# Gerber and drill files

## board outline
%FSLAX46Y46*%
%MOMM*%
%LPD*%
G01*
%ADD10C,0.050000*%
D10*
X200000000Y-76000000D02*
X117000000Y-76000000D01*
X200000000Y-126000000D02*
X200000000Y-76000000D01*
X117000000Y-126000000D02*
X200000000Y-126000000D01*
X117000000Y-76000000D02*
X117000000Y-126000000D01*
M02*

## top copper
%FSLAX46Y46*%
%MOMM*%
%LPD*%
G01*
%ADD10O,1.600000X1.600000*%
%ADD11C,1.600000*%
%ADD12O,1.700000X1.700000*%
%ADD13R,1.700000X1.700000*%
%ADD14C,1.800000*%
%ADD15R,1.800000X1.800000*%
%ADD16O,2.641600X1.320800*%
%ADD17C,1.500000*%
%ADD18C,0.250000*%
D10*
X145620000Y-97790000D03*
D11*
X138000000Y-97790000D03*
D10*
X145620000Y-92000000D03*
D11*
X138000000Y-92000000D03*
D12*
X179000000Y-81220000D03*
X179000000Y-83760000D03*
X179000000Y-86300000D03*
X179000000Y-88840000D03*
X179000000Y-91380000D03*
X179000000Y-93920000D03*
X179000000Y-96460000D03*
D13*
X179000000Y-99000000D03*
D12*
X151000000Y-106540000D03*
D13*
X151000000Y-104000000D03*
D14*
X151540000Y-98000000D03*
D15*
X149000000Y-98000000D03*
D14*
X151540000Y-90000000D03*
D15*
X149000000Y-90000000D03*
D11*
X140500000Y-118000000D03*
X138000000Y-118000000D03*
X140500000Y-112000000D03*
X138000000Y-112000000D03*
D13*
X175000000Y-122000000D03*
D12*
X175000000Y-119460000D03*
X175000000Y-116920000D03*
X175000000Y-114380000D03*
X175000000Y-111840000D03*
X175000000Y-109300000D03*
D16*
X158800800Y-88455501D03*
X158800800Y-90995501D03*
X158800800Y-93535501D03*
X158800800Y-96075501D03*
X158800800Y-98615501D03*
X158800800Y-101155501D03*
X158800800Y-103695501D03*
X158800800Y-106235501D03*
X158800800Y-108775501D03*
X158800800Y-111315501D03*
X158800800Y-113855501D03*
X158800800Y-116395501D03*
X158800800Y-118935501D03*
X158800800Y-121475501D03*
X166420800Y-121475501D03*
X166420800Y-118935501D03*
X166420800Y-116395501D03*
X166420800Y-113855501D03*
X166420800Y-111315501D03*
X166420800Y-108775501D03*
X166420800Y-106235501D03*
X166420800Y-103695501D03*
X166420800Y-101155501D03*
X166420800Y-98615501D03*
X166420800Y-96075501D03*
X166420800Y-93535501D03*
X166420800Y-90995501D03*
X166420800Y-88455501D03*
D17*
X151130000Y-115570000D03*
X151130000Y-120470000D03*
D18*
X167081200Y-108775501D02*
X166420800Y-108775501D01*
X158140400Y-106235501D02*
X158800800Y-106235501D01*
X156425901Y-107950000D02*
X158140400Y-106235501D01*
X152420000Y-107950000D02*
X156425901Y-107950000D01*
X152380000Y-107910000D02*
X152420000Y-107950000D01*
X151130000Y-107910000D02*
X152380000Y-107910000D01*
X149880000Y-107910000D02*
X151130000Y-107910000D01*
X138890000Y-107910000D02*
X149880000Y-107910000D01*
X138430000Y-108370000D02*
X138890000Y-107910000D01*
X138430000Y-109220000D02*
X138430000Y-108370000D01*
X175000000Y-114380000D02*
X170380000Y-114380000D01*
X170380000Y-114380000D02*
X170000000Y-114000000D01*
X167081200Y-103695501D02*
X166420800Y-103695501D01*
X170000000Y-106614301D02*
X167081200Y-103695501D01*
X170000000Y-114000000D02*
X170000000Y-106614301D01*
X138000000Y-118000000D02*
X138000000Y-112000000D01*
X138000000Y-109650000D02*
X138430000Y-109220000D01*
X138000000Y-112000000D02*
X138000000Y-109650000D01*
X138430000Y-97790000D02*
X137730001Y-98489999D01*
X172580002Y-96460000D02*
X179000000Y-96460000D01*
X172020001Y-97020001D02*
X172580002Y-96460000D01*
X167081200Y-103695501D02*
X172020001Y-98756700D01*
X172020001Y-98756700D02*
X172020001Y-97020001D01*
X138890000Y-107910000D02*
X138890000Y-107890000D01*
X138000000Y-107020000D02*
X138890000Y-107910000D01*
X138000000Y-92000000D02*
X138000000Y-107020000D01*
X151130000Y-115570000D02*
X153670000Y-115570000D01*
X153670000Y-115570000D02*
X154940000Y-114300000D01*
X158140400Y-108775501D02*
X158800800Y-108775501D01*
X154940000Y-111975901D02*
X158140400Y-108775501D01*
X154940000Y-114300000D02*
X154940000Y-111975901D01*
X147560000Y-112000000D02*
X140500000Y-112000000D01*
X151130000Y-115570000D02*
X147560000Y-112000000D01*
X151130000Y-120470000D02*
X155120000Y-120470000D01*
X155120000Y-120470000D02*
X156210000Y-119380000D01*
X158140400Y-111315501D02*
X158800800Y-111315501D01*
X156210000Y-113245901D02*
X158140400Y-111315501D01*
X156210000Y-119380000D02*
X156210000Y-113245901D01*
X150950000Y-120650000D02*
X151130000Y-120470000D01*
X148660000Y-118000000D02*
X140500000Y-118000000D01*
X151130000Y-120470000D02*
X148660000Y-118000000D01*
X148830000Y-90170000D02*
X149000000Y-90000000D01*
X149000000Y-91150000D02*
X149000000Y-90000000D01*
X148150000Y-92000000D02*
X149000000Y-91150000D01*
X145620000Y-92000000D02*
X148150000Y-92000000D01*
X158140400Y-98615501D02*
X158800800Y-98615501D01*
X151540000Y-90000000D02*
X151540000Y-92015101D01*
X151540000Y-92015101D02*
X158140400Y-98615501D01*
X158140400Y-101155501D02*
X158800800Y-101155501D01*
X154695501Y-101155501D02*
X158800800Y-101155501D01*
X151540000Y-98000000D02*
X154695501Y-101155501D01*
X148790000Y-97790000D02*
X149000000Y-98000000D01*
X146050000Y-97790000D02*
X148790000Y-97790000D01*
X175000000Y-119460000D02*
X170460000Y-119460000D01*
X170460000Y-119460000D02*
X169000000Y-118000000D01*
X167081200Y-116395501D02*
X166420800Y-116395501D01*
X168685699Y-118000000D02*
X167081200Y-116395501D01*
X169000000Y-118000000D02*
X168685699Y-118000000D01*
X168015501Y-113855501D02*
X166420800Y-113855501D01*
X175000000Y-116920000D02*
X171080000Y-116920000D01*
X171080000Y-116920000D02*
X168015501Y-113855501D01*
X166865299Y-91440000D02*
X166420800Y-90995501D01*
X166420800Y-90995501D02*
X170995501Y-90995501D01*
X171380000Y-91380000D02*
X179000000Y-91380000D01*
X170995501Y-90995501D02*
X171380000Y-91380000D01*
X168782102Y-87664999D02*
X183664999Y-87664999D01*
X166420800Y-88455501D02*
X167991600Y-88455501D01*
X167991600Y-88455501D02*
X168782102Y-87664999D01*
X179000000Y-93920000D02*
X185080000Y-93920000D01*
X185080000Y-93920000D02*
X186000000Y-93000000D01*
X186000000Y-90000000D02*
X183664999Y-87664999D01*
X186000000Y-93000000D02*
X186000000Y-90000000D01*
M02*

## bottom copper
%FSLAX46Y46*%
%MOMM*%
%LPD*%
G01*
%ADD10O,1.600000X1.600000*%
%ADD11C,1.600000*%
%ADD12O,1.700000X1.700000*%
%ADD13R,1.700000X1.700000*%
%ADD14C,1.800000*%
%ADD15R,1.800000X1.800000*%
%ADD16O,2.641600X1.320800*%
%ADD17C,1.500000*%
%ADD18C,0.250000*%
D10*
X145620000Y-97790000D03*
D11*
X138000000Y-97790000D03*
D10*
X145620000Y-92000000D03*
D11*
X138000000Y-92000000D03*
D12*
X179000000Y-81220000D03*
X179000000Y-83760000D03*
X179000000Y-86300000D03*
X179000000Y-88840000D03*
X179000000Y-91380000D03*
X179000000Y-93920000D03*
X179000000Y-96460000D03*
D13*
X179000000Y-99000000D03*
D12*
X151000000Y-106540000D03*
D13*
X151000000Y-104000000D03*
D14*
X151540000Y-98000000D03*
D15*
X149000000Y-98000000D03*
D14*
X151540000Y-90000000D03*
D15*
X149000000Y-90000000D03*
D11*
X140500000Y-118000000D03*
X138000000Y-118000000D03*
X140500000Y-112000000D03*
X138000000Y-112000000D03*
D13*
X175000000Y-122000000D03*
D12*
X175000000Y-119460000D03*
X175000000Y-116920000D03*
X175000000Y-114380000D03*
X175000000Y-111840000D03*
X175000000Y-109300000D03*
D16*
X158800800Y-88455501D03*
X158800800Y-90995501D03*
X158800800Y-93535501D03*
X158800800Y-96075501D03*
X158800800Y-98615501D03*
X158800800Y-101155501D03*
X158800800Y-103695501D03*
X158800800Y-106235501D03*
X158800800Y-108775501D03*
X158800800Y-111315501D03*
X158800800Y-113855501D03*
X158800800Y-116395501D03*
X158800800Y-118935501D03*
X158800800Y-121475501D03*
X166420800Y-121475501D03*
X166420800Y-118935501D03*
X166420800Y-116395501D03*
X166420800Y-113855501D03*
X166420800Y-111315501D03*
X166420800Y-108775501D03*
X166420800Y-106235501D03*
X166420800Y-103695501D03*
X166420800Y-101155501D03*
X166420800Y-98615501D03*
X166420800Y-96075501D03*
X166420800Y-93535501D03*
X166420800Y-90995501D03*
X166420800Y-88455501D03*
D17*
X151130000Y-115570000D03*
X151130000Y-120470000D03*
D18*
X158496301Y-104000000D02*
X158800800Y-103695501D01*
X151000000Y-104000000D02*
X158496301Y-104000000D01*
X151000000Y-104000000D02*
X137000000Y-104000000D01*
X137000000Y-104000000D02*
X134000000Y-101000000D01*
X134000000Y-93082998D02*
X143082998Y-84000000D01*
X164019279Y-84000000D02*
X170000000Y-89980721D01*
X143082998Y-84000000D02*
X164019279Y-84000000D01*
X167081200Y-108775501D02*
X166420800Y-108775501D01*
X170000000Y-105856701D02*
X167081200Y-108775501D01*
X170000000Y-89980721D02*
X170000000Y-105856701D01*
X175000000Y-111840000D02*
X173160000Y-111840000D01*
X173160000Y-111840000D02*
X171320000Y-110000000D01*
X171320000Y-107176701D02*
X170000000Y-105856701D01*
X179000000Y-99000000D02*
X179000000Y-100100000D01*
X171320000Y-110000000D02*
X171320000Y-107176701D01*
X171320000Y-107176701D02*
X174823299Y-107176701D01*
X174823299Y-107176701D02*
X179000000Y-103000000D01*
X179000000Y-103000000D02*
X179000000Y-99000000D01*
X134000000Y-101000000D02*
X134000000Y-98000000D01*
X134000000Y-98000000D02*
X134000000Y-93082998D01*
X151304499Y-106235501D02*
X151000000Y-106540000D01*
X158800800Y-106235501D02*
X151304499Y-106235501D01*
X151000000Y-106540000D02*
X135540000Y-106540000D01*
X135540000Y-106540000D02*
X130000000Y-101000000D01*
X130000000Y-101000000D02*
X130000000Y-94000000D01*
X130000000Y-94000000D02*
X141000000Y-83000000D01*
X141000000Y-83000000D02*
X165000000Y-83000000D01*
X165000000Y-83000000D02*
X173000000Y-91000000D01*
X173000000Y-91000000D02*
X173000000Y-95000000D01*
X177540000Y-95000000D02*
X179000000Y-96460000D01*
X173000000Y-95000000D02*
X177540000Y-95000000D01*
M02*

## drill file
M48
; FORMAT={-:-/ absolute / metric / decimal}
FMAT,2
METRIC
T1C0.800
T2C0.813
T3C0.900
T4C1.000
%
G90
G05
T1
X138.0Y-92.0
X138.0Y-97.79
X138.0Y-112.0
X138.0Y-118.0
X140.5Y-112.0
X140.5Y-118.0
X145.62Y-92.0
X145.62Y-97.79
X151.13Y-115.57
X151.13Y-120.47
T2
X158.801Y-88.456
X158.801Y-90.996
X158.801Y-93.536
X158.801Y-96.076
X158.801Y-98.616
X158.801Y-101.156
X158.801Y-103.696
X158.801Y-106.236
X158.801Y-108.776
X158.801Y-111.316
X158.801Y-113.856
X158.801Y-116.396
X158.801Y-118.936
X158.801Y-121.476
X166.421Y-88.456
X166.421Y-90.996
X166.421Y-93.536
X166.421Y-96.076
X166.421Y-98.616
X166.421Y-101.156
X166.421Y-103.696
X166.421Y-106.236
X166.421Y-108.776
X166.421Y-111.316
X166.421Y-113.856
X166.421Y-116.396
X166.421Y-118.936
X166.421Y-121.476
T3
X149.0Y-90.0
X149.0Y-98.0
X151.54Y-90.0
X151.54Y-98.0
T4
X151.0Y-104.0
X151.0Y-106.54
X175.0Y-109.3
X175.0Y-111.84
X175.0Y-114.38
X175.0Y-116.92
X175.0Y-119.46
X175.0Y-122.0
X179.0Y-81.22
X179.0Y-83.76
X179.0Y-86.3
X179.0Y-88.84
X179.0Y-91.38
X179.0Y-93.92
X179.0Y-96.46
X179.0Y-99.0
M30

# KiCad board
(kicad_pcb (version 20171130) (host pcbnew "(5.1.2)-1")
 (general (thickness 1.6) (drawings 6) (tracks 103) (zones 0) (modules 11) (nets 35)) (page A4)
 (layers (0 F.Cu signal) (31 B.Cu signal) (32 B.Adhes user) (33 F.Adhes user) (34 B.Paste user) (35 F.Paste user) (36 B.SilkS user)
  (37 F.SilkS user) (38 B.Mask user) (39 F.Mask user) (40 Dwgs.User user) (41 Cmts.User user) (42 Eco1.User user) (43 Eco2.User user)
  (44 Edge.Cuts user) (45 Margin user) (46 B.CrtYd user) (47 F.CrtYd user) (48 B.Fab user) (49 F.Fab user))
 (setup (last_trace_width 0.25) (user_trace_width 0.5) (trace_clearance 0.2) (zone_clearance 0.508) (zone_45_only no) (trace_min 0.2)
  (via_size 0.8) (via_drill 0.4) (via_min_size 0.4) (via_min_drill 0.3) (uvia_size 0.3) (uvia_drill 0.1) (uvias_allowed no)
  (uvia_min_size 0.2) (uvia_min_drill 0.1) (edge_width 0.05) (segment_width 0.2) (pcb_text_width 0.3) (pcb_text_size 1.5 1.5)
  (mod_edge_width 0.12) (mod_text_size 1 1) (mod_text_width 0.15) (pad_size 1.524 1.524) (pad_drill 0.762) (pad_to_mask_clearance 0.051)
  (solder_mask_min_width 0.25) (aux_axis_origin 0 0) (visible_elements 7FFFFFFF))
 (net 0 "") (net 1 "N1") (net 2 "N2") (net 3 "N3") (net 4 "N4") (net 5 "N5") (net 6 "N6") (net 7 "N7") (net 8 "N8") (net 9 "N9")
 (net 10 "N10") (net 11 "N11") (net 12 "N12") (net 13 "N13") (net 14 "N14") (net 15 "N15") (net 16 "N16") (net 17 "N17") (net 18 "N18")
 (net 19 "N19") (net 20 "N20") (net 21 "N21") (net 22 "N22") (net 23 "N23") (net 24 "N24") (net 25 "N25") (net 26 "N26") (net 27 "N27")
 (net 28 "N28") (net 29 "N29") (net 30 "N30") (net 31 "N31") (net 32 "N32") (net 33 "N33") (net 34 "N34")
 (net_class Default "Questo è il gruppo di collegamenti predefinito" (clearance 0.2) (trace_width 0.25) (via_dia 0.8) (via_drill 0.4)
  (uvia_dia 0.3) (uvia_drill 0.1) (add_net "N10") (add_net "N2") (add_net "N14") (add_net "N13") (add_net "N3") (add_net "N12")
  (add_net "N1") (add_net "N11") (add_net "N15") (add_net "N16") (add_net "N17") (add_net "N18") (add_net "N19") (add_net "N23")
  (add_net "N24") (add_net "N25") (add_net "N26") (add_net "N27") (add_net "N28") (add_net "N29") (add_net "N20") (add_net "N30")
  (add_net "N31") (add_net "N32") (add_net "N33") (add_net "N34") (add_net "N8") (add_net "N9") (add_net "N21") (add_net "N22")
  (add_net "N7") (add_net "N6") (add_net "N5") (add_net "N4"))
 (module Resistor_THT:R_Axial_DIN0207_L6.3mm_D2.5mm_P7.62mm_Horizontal (layer F.Cu) (at 138 97.79)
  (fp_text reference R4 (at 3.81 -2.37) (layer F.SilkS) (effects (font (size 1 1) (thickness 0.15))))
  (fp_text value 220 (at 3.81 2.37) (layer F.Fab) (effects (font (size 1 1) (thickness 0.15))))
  (pad 2 thru_hole oval (at 7.62 0) (size 1.6 1.6) (drill 0.8) (layers *.Cu *.Mask) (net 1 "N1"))
  (pad 1 thru_hole circle (at 0 0) (size 1.6 1.6) (drill 0.8) (layers *.Cu *.Mask) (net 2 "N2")))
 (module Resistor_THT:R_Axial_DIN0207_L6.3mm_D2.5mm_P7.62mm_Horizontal (layer F.Cu) (at 138 92)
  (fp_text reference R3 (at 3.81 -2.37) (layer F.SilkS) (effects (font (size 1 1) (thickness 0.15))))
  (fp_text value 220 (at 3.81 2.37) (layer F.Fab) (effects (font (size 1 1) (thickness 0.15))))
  (pad 2 thru_hole oval (at 7.62 0) (size 1.6 1.6) (drill 0.8) (layers *.Cu *.Mask) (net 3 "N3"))
  (pad 1 thru_hole circle (at 0 0) (size 1.6 1.6) (drill 0.8) (layers *.Cu *.Mask) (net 2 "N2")))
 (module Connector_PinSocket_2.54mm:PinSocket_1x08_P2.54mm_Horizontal (layer F.Cu) (at 179 99 180)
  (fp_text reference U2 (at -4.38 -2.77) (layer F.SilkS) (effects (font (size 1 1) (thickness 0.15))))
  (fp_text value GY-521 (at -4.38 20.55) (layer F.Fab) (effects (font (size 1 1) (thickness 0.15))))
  (pad 8 thru_hole oval (at 0 17.78 180) (size 1.7 1.7) (drill 1) (layers *.Cu *.Mask) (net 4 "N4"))
  (pad 7 thru_hole oval (at 0 15.24 180) (size 1.7 1.7) (drill 1) (layers *.Cu *.Mask) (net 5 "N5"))
  (pad 6 thru_hole oval (at 0 12.7 180) (size 1.7 1.7) (drill 1) (layers *.Cu *.Mask) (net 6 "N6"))
  (pad 5 thru_hole oval (at 0 10.16 180) (size 1.7 1.7) (drill 1) (layers *.Cu *.Mask) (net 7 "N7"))
  (pad 4 thru_hole oval (at 0 7.62 180) (size 1.7 1.7) (drill 1) (layers *.Cu *.Mask) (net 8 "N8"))
  (pad 3 thru_hole oval (at 0 5.08 180) (size 1.7 1.7) (drill 1) (layers *.Cu *.Mask) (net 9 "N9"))
  (pad 2 thru_hole oval (at 0 2.54 180) (size 1.7 1.7) (drill 1) (layers *.Cu *.Mask) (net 2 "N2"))
  (pad 1 thru_hole rect (at 0 0 180) (size 1.7 1.7) (drill 1) (layers *.Cu *.Mask) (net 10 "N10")))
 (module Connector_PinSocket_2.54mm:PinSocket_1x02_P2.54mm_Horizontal (layer F.Cu) (at 151 104)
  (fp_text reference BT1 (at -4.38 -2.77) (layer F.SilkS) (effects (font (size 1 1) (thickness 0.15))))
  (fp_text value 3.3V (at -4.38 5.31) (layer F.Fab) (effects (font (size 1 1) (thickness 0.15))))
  (pad 2 thru_hole oval (at 0 2.54) (size 1.7 1.7) (drill 1) (layers *.Cu *.Mask) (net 2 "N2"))
  (pad 1 thru_hole rect (at 0 0) (size 1.7 1.7) (drill 1) (layers *.Cu *.Mask) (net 10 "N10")))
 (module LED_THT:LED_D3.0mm (layer F.Cu) (at 149 98)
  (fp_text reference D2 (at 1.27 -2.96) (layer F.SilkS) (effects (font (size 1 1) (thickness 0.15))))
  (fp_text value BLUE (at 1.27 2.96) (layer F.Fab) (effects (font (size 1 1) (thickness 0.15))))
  (pad 2 thru_hole circle (at 2.54 0) (size 1.8 1.8) (drill 0.9) (layers *.Cu *.Mask) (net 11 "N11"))
  (pad 1 thru_hole rect (at 0 0) (size 1.8 1.8) (drill 0.9) (layers *.Cu *.Mask) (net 1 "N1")))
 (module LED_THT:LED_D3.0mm (layer F.Cu) (at 149 90)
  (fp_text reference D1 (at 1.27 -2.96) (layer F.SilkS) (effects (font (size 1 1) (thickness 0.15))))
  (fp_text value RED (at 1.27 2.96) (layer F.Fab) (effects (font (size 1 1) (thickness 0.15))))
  (pad 2 thru_hole circle (at 2.54 0) (size 1.8 1.8) (drill 0.9) (layers *.Cu *.Mask) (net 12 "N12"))
  (pad 1 thru_hole rect (at 0 0) (size 1.8 1.8) (drill 0.9) (layers *.Cu *.Mask) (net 3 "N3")))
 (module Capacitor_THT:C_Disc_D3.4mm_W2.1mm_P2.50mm (layer F.Cu) (at 138 118)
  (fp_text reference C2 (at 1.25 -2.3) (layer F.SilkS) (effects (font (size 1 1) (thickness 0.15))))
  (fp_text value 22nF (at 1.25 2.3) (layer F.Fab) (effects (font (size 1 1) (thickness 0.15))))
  (pad 2 thru_hole circle (at 2.5 0) (size 1.6 1.6) (drill 0.8) (layers *.Cu *.Mask) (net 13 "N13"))
  (pad 1 thru_hole circle (at 0 0) (size 1.6 1.6) (drill 0.8) (layers *.Cu *.Mask) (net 2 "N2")))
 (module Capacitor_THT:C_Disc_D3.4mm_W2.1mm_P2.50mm (layer F.Cu) (at 138 112)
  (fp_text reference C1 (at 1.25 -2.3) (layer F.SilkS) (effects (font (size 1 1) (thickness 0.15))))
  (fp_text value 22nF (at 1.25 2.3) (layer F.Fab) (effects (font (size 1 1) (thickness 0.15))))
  (pad 2 thru_hole circle (at 2.5 0) (size 1.6 1.6) (drill 0.8) (layers *.Cu *.Mask) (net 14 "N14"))
  (pad 1 thru_hole circle (at 0 0) (size 1.6 1.6) (drill 0.8) (layers *.Cu *.Mask) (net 2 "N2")))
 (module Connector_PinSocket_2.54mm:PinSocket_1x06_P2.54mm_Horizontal (layer F.Cu) (at 175 122 180)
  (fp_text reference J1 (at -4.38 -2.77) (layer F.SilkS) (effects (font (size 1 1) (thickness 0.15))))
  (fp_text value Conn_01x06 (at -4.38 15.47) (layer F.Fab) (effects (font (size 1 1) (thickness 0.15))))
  (pad 1 thru_hole rect (at 0 0 180) (size 1.7 1.7) (drill 1) (layers *.Cu *.Mask) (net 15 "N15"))
  (pad 2 thru_hole oval (at 0 2.54 180) (size 1.7 1.7) (drill 1) (layers *.Cu *.Mask) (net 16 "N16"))
  (pad 3 thru_hole oval (at 0 5.08 180) (size 1.7 1.7) (drill 1) (layers *.Cu *.Mask) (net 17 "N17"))
  (pad 4 thru_hole oval (at 0 7.62 180) (size 1.7 1.7) (drill 1) (layers *.Cu *.Mask) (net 2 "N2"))
  (pad 5 thru_hole oval (at 0 10.16 180) (size 1.7 1.7) (drill 1) (layers *.Cu *.Mask) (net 10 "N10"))
  (pad 6 thru_hole oval (at 0 12.7 180) (size 1.7 1.7) (drill 1) (layers *.Cu *.Mask) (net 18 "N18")))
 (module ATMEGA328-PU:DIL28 (layer F.Cu) (at 162.6108 104.965501)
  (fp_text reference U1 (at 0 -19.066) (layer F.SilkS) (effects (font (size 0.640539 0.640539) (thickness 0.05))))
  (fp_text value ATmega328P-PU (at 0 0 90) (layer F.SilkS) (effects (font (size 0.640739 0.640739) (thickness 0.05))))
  (pad 1 thru_hole oval (at -3.81 -16.51) (size 2.6416 1.3208) (drill 0.8128) (layers *.Cu *.Mask) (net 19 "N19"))
  (pad 2 thru_hole oval (at -3.81 -13.97) (size 2.6416 1.3208) (drill 0.8128) (layers *.Cu *.Mask) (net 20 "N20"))
  (pad 3 thru_hole oval (at -3.81 -11.43) (size 2.6416 1.3208) (drill 0.8128) (layers *.Cu *.Mask) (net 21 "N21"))
  (pad 4 thru_hole oval (at -3.81 -8.89) (size 2.6416 1.3208) (drill 0.8128) (layers *.Cu *.Mask) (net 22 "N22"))
  (pad 5 thru_hole oval (at -3.81 -6.35) (size 2.6416 1.3208) (drill 0.8128) (layers *.Cu *.Mask) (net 12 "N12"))
  (pad 6 thru_hole oval (at -3.81 -3.81) (size 2.6416 1.3208) (drill 0.8128) (layers *.Cu *.Mask) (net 11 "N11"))
  (pad 7 thru_hole oval (at -3.81 -1.27) (size 2.6416 1.3208) (drill 0.8128) (layers *.Cu *.Mask) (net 10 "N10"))
  (pad 8 thru_hole oval (at -3.81 1.27) (size 2.6416 1.3208) (drill 0.8128) (layers *.Cu *.Mask) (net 2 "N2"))
  (pad 9 thru_hole oval (at -3.81 3.81) (size 2.6416 1.3208) (drill 0.8128) (layers *.Cu *.Mask) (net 14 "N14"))
  (pad 10 thru_hole oval (at -3.81 6.35) (size 2.6416 1.3208) (drill 0.8128) (layers *.Cu *.Mask) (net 13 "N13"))
  (pad 11 thru_hole oval (at -3.81 8.89) (size 2.6416 1.3208) (drill 0.8128) (layers *.Cu *.Mask) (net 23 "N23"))
  (pad 12 thru_hole oval (at -3.81 11.43) (size 2.6416 1.3208) (drill 0.8128) (layers *.Cu *.Mask) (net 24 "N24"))
  (pad 13 thru_hole oval (at -3.81 13.97) (size 2.6416 1.3208) (drill 0.8128) (layers *.Cu *.Mask) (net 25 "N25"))
  (pad 14 thru_hole oval (at -3.81 16.51) (size 2.6416 1.3208) (drill 0.8128) (layers *.Cu *.Mask) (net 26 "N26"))
  (pad 15 thru_hole oval (at 3.81 16.51) (size 2.6416 1.3208) (drill 0.8128) (layers *.Cu *.Mask) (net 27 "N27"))
  (pad 16 thru_hole oval (at 3.81 13.97) (size 2.6416 1.3208) (drill 0.8128) (layers *.Cu *.Mask) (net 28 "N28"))
  (pad 17 thru_hole oval (at 3.81 11.43) (size 2.6416 1.3208) (drill 0.8128) (layers *.Cu *.Mask) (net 16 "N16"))
  (pad 18 thru_hole oval (at 3.81 8.89) (size 2.6416 1.3208) (drill 0.8128) (layers *.Cu *.Mask) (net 17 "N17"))
  (pad 19 thru_hole oval (at 3.81 6.35) (size 2.6416 1.3208) (drill 0.8128) (layers *.Cu *.Mask) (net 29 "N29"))
  (pad 20 thru_hole oval (at 3.81 3.81) (size 2.6416 1.3208) (drill 0.8128) (layers *.Cu *.Mask) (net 10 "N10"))
  (pad 21 thru_hole oval (at 3.81 1.27) (size 2.6416 1.3208) (drill 0.8128) (layers *.Cu *.Mask) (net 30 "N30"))
  (pad 22 thru_hole oval (at 3.81 -1.27) (size 2.6416 1.3208) (drill 0.8128) (layers *.Cu *.Mask) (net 2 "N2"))
  (pad 23 thru_hole oval (at 3.81 -3.81) (size 2.6416 1.3208) (drill 0.8128) (layers *.Cu *.Mask) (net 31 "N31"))
  (pad 24 thru_hole oval (at 3.81 -6.35) (size 2.6416 1.3208) (drill 0.8128) (layers *.Cu *.Mask) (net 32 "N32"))
  (pad 25 thru_hole oval (at 3.81 -8.89) (size 2.6416 1.3208) (drill 0.8128) (layers *.Cu *.Mask) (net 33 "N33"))
  (pad 26 thru_hole oval (at 3.81 -11.43) (size 2.6416 1.3208) (drill 0.8128) (layers *.Cu *.Mask) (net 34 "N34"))
  (pad 27 thru_hole oval (at 3.81 -13.97) (size 2.6416 1.3208) (drill 0.8128) (layers *.Cu *.Mask) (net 8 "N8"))
  (pad 28 thru_hole oval (at 3.81 -16.51) (size 2.6416 1.3208) (drill 0.8128) (layers *.Cu *.Mask) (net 9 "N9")))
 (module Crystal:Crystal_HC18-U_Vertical (layer F.Cu) (at 151.13 115.57 270)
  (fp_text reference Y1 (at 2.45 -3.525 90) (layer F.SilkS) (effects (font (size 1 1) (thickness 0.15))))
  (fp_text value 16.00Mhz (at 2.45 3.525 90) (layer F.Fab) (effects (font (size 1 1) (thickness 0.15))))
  (pad 1 thru_hole circle (at 0 0 270) (size 1.5 1.5) (drill 0.8) (layers *.Cu *.Mask) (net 14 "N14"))
  (pad 2 thru_hole circle (at 4.9 0 270) (size 1.5 1.5) (drill 0.8) (layers *.Cu *.Mask) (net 13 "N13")))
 (gr_line (start 200 76) (end 117 76) (layer Edge.Cuts) (width 0.05))
 (gr_line (start 200 126) (end 200 76) (layer Edge.Cuts) (width 0.05))
 (gr_line (start 117 126) (end 200 126) (layer Edge.Cuts) (width 0.05))
 (gr_line (start 117 76) (end 117 126) (layer Edge.Cuts) (width 0.05))
 (segment (start 158.496301 104) (end 158.8008 103.695501) (width 0.25) (layer B.Cu) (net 10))
 (segment (start 151 104) (end 158.496301 104) (width 0.25) (layer B.Cu) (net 10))
 (segment (start 151 104) (end 137 104) (width 0.25) (layer B.Cu) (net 10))
 (segment (start 137 104) (end 134 101) (width 0.25) (layer B.Cu) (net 10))
 (segment (start 134 93.082998) (end 143.082998 84) (width 0.25) (layer B.Cu) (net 10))
 (segment (start 164.019279 84) (end 170 89.980721) (width 0.25) (layer B.Cu) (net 10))
 (segment (start 143.082998 84) (end 164.019279 84) (width 0.25) (layer B.Cu) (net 10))
 (segment (start 167.0812 108.775501) (end 166.4208 108.775501) (width 0.25) (layer B.Cu) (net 10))
 (segment (start 170 105.856701) (end 167.0812 108.775501) (width 0.25) (layer B.Cu) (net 10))
 (segment (start 170 89.980721) (end 170 105.856701) (width 0.25) (layer B.Cu) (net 10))
 (segment (start 175 111.84) (end 173.16 111.84) (width 0.25) (layer B.Cu) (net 10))
 (segment (start 173.16 111.84) (end 171.32 110) (width 0.25) (layer B.Cu) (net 10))
 (segment (start 171.32 107.176701) (end 170 105.856701) (width 0.25) (layer B.Cu) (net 10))
 (segment (start 167.0812 108.775501) (end 166.4208 108.775501) (width 0.25) (layer F.Cu) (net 10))
 (segment (start 179 99) (end 179 100.1) (width 0.25) (layer B.Cu) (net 10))
 (segment (start 171.32 110) (end 171.32 107.176701) (width 0.25) (layer B.Cu) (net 10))
 (segment (start 171.32 107.176701) (end 174.823299 107.176701) (width 0.25) (layer B.Cu) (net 10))
 (segment (start 174.823299 107.176701) (end 179 103) (width 0.25) (layer B.Cu) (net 10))
 (segment (start 179 103) (end 179 99) (width 0.25) (layer B.Cu) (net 10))
 (segment (start 134 101) (end 134 98) (width 0.25) (layer B.Cu) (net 10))
 (segment (start 134 98) (end 134 93.082998) (width 0.25) (layer B.Cu) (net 10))
 (segment (start 158.1404 106.235501) (end 158.8008 106.235501) (width 0.25) (layer F.Cu) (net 2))
 (segment (start 156.425901 107.95) (end 158.1404 106.235501) (width 0.25) (layer F.Cu) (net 2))
 (segment (start 152.42 107.95) (end 156.425901 107.95) (width 0.25) (layer F.Cu) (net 2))
 (segment (start 152.38 107.91) (end 152.42 107.95) (width 0.25) (layer F.Cu) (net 2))
 (segment (start 151.13 107.91) (end 152.38 107.91) (width 0.25) (layer F.Cu) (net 2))
 (segment (start 149.88 107.91) (end 151.13 107.91) (width 0.25) (layer F.Cu) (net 2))
 (segment (start 138.89 107.91) (end 149.88 107.91) (width 0.25) (layer F.Cu) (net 2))
 (segment (start 138.43 108.37) (end 138.89 107.91) (width 0.25) (layer F.Cu) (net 2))
 (segment (start 138.43 109.22) (end 138.43 108.37) (width 0.25) (layer F.Cu) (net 2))
 (segment (start 175 114.38) (end 170.38 114.38) (width 0.25) (layer F.Cu) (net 2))
 (segment (start 170.38 114.38) (end 170 114) (width 0.25) (layer F.Cu) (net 2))
 (segment (start 167.0812 103.695501) (end 166.4208 103.695501) (width 0.25) (layer F.Cu) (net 2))
 (segment (start 170 106.614301) (end 167.0812 103.695501) (width 0.25) (layer F.Cu) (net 2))
 (segment (start 170 114) (end 170 106.614301) (width 0.25) (layer F.Cu) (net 2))
 (segment (start 138 118) (end 138 112) (width 0.25) (layer F.Cu) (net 2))
 (segment (start 138 109.65) (end 138.43 109.22) (width 0.25) (layer F.Cu) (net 2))
 (segment (start 138 112) (end 138 109.65) (width 0.25) (layer F.Cu) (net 2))
 (segment (start 138.43 97.79) (end 137.730001 98.489999) (width 0.25) (layer F.Cu) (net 2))
 (segment (start 172.580002 96.46) (end 179 96.46) (width 0.25) (layer F.Cu) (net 2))
 (segment (start 172.020001 97.020001) (end 172.580002 96.46) (width 0.25) (layer F.Cu) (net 2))
 (segment (start 167.0812 103.695501) (end 172.020001 98.7567) (width 0.25) (layer F.Cu) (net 2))
 (segment (start 172.020001 98.7567) (end 172.020001 97.020001) (width 0.25) (layer F.Cu) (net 2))
 (segment (start 151.304499 106.235501) (end 151 106.54) (width 0.25) (layer B.Cu) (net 2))
 (segment (start 158.8008 106.235501) (end 151.304499 106.235501) (width 0.25) (layer B.Cu) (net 2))
 (segment (start 151 106.54) (end 135.54 106.54) (width 0.25) (layer B.Cu) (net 2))
 (segment (start 135.54 106.54) (end 130 101) (width 0.25) (layer B.Cu) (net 2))
 (segment (start 130 101) (end 130 94) (width 0.25) (layer B.Cu) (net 2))
 (segment (start 130 94) (end 141 83) (width 0.25) (layer B.Cu) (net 2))
 (segment (start 141 83) (end 165 83) (width 0.25) (layer B.Cu) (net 2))
 (segment (start 165 83) (end 173 91) (width 0.25) (layer B.Cu) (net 2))
 (segment (start 173 91) (end 173 95) (width 0.25) (layer B.Cu) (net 2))
 (segment (start 177.54 95) (end 179 96.46) (width 0.25) (layer B.Cu) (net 2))
 (segment (start 173 95) (end 177.54 95) (width 0.25) (layer B.Cu) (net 2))
 (segment (start 138.89 107.91) (end 138.89 107.89) (width 0.25) (layer F.Cu) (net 2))
 (segment (start 138 107.02) (end 138.89 107.91) (width 0.25) (layer F.Cu) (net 2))
 (segment (start 138 92) (end 138 107.02) (width 0.25) (layer F.Cu) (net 2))
 (segment (start 151.13 115.57) (end 153.67 115.57) (width 0.25) (layer F.Cu) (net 14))
 (segment (start 153.67 115.57) (end 154.94 114.3) (width 0.25) (layer F.Cu) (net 14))
 (segment (start 158.1404 108.775501) (end 158.8008 108.775501) (width 0.25) (layer F.Cu) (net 14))
 (segment (start 154.94 111.975901) (end 158.1404 108.775501) (width 0.25) (layer F.Cu) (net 14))
 (segment (start 154.94 114.3) (end 154.94 111.975901) (width 0.25) (layer F.Cu) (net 14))
 (segment (start 147.56 112) (end 140.5 112) (width 0.25) (layer F.Cu) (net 14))
 (segment (start 151.13 115.57) (end 147.56 112) (width 0.25) (layer F.Cu) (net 14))
 (segment (start 151.13 120.47) (end 155.12 120.47) (width 0.25) (layer F.Cu) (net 13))
 (segment (start 155.12 120.47) (end 156.21 119.38) (width 0.25) (layer F.Cu) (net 13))
 (segment (start 158.1404 111.315501) (end 158.8008 111.315501) (width 0.25) (layer F.Cu) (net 13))
 (segment (start 156.21 113.245901) (end 158.1404 111.315501) (width 0.25) (layer F.Cu) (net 13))
 (segment (start 156.21 119.38) (end 156.21 113.245901) (width 0.25) (layer F.Cu) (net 13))
 (segment (start 150.95 120.65) (end 151.13 120.47) (width 0.25) (layer F.Cu) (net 13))
 (segment (start 148.66 118) (end 140.5 118) (width 0.25) (layer F.Cu) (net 13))
 (segment (start 151.13 120.47) (end 148.66 118) (width 0.25) (layer F.Cu) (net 13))
 (segment (start 148.83 90.17) (end 149 90) (width 0.25) (layer F.Cu) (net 3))
 (segment (start 149 91.15) (end 149 90) (width 0.25) (layer F.Cu) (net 3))
 (segment (start 148.15 92) (end 149 91.15) (width 0.25) (layer F.Cu) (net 3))
 (segment (start 145.62 92) (end 148.15 92) (width 0.25) (layer F.Cu) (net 3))
 (segment (start 158.1404 98.615501) (end 158.8008 98.615501) (width 0.25) (layer F.Cu) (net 12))
 (segment (start 151.54 90) (end 151.54 92.015101) (width 0.25) (layer F.Cu) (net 12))
 (segment (start 151.54 92.015101) (end 158.1404 98.615501) (width 0.25) (layer F.Cu) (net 12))
 (segment (start 158.1404 101.155501) (end 158.8008 101.155501) (width 0.25) (layer F.Cu) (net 11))
 (segment (start 154.695501 101.155501) (end 158.8008 101.155501) (width 0.25) (layer F.Cu) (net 11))
 (segment (start 151.54 98) (end 154.695501 101.155501) (width 0.25) (layer F.Cu) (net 11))
 (segment (start 148.79 97.79) (end 149 98) (width 0.25) (layer F.Cu) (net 1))
 (segment (start 146.05 97.79) (end 148.79 97.79) (width 0.25) (layer F.Cu) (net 1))
 (segment (start 175 119.46) (end 170.46 119.46) (width 0.25) (layer F.Cu) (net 16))
 (segment (start 170.46 119.46) (end 169 118) (width 0.25) (layer F.Cu) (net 16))
 (segment (start 167.0812 116.395501) (end 166.4208 116.395501) (width 0.25) (layer F.Cu) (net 16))
 (segment (start 168.685699 118) (end 167.0812 116.395501) (width 0.25) (layer F.Cu) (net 16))
 (segment (start 169 118) (end 168.685699 118) (width 0.25) (layer F.Cu) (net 16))
 (segment (start 168.015501 113.855501) (end 166.4208 113.855501) (width 0.25) (layer F.Cu) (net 17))
 (segment (start 175 116.92) (end 171.08 116.92) (width 0.25) (layer F.Cu) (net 17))
 (segment (start 171.08 116.92) (end 168.015501 113.855501) (width 0.25) (layer F.Cu) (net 17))
 (segment (start 166.865299 91.44) (end 166.4208 90.995501) (width 0.25) (layer F.Cu) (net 8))
 (segment (start 166.4208 90.995501) (end 170.995501 90.995501) (width 0.25) (layer F.Cu) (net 8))
 (segment (start 171.38 91.38) (end 179 91.38) (width 0.25) (layer F.Cu) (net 8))
 (segment (start 170.995501 90.995501) (end 171.38 91.38) (width 0.25) (layer F.Cu) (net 8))
 (segment (start 168.782102 87.664999) (end 183.664999 87.664999) (width 0.25) (layer F.Cu) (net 9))
 (segment (start 166.4208 88.455501) (end 167.9916 88.455501) (width 0.25) (layer F.Cu) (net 9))
 (segment (start 167.9916 88.455501) (end 168.782102 87.664999) (width 0.25) (layer F.Cu) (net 9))
 (segment (start 179 93.92) (end 185.08 93.92) (width 0.25) (layer F.Cu) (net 9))
 (segment (start 185.08 93.92) (end 186 93) (width 0.25) (layer F.Cu) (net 9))
 (segment (start 186 90) (end 183.664999 87.664999) (width 0.25) (layer F.Cu) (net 9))
 (segment (start 186 93) (end 186 90) (width 0.25) (layer F.Cu) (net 9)))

